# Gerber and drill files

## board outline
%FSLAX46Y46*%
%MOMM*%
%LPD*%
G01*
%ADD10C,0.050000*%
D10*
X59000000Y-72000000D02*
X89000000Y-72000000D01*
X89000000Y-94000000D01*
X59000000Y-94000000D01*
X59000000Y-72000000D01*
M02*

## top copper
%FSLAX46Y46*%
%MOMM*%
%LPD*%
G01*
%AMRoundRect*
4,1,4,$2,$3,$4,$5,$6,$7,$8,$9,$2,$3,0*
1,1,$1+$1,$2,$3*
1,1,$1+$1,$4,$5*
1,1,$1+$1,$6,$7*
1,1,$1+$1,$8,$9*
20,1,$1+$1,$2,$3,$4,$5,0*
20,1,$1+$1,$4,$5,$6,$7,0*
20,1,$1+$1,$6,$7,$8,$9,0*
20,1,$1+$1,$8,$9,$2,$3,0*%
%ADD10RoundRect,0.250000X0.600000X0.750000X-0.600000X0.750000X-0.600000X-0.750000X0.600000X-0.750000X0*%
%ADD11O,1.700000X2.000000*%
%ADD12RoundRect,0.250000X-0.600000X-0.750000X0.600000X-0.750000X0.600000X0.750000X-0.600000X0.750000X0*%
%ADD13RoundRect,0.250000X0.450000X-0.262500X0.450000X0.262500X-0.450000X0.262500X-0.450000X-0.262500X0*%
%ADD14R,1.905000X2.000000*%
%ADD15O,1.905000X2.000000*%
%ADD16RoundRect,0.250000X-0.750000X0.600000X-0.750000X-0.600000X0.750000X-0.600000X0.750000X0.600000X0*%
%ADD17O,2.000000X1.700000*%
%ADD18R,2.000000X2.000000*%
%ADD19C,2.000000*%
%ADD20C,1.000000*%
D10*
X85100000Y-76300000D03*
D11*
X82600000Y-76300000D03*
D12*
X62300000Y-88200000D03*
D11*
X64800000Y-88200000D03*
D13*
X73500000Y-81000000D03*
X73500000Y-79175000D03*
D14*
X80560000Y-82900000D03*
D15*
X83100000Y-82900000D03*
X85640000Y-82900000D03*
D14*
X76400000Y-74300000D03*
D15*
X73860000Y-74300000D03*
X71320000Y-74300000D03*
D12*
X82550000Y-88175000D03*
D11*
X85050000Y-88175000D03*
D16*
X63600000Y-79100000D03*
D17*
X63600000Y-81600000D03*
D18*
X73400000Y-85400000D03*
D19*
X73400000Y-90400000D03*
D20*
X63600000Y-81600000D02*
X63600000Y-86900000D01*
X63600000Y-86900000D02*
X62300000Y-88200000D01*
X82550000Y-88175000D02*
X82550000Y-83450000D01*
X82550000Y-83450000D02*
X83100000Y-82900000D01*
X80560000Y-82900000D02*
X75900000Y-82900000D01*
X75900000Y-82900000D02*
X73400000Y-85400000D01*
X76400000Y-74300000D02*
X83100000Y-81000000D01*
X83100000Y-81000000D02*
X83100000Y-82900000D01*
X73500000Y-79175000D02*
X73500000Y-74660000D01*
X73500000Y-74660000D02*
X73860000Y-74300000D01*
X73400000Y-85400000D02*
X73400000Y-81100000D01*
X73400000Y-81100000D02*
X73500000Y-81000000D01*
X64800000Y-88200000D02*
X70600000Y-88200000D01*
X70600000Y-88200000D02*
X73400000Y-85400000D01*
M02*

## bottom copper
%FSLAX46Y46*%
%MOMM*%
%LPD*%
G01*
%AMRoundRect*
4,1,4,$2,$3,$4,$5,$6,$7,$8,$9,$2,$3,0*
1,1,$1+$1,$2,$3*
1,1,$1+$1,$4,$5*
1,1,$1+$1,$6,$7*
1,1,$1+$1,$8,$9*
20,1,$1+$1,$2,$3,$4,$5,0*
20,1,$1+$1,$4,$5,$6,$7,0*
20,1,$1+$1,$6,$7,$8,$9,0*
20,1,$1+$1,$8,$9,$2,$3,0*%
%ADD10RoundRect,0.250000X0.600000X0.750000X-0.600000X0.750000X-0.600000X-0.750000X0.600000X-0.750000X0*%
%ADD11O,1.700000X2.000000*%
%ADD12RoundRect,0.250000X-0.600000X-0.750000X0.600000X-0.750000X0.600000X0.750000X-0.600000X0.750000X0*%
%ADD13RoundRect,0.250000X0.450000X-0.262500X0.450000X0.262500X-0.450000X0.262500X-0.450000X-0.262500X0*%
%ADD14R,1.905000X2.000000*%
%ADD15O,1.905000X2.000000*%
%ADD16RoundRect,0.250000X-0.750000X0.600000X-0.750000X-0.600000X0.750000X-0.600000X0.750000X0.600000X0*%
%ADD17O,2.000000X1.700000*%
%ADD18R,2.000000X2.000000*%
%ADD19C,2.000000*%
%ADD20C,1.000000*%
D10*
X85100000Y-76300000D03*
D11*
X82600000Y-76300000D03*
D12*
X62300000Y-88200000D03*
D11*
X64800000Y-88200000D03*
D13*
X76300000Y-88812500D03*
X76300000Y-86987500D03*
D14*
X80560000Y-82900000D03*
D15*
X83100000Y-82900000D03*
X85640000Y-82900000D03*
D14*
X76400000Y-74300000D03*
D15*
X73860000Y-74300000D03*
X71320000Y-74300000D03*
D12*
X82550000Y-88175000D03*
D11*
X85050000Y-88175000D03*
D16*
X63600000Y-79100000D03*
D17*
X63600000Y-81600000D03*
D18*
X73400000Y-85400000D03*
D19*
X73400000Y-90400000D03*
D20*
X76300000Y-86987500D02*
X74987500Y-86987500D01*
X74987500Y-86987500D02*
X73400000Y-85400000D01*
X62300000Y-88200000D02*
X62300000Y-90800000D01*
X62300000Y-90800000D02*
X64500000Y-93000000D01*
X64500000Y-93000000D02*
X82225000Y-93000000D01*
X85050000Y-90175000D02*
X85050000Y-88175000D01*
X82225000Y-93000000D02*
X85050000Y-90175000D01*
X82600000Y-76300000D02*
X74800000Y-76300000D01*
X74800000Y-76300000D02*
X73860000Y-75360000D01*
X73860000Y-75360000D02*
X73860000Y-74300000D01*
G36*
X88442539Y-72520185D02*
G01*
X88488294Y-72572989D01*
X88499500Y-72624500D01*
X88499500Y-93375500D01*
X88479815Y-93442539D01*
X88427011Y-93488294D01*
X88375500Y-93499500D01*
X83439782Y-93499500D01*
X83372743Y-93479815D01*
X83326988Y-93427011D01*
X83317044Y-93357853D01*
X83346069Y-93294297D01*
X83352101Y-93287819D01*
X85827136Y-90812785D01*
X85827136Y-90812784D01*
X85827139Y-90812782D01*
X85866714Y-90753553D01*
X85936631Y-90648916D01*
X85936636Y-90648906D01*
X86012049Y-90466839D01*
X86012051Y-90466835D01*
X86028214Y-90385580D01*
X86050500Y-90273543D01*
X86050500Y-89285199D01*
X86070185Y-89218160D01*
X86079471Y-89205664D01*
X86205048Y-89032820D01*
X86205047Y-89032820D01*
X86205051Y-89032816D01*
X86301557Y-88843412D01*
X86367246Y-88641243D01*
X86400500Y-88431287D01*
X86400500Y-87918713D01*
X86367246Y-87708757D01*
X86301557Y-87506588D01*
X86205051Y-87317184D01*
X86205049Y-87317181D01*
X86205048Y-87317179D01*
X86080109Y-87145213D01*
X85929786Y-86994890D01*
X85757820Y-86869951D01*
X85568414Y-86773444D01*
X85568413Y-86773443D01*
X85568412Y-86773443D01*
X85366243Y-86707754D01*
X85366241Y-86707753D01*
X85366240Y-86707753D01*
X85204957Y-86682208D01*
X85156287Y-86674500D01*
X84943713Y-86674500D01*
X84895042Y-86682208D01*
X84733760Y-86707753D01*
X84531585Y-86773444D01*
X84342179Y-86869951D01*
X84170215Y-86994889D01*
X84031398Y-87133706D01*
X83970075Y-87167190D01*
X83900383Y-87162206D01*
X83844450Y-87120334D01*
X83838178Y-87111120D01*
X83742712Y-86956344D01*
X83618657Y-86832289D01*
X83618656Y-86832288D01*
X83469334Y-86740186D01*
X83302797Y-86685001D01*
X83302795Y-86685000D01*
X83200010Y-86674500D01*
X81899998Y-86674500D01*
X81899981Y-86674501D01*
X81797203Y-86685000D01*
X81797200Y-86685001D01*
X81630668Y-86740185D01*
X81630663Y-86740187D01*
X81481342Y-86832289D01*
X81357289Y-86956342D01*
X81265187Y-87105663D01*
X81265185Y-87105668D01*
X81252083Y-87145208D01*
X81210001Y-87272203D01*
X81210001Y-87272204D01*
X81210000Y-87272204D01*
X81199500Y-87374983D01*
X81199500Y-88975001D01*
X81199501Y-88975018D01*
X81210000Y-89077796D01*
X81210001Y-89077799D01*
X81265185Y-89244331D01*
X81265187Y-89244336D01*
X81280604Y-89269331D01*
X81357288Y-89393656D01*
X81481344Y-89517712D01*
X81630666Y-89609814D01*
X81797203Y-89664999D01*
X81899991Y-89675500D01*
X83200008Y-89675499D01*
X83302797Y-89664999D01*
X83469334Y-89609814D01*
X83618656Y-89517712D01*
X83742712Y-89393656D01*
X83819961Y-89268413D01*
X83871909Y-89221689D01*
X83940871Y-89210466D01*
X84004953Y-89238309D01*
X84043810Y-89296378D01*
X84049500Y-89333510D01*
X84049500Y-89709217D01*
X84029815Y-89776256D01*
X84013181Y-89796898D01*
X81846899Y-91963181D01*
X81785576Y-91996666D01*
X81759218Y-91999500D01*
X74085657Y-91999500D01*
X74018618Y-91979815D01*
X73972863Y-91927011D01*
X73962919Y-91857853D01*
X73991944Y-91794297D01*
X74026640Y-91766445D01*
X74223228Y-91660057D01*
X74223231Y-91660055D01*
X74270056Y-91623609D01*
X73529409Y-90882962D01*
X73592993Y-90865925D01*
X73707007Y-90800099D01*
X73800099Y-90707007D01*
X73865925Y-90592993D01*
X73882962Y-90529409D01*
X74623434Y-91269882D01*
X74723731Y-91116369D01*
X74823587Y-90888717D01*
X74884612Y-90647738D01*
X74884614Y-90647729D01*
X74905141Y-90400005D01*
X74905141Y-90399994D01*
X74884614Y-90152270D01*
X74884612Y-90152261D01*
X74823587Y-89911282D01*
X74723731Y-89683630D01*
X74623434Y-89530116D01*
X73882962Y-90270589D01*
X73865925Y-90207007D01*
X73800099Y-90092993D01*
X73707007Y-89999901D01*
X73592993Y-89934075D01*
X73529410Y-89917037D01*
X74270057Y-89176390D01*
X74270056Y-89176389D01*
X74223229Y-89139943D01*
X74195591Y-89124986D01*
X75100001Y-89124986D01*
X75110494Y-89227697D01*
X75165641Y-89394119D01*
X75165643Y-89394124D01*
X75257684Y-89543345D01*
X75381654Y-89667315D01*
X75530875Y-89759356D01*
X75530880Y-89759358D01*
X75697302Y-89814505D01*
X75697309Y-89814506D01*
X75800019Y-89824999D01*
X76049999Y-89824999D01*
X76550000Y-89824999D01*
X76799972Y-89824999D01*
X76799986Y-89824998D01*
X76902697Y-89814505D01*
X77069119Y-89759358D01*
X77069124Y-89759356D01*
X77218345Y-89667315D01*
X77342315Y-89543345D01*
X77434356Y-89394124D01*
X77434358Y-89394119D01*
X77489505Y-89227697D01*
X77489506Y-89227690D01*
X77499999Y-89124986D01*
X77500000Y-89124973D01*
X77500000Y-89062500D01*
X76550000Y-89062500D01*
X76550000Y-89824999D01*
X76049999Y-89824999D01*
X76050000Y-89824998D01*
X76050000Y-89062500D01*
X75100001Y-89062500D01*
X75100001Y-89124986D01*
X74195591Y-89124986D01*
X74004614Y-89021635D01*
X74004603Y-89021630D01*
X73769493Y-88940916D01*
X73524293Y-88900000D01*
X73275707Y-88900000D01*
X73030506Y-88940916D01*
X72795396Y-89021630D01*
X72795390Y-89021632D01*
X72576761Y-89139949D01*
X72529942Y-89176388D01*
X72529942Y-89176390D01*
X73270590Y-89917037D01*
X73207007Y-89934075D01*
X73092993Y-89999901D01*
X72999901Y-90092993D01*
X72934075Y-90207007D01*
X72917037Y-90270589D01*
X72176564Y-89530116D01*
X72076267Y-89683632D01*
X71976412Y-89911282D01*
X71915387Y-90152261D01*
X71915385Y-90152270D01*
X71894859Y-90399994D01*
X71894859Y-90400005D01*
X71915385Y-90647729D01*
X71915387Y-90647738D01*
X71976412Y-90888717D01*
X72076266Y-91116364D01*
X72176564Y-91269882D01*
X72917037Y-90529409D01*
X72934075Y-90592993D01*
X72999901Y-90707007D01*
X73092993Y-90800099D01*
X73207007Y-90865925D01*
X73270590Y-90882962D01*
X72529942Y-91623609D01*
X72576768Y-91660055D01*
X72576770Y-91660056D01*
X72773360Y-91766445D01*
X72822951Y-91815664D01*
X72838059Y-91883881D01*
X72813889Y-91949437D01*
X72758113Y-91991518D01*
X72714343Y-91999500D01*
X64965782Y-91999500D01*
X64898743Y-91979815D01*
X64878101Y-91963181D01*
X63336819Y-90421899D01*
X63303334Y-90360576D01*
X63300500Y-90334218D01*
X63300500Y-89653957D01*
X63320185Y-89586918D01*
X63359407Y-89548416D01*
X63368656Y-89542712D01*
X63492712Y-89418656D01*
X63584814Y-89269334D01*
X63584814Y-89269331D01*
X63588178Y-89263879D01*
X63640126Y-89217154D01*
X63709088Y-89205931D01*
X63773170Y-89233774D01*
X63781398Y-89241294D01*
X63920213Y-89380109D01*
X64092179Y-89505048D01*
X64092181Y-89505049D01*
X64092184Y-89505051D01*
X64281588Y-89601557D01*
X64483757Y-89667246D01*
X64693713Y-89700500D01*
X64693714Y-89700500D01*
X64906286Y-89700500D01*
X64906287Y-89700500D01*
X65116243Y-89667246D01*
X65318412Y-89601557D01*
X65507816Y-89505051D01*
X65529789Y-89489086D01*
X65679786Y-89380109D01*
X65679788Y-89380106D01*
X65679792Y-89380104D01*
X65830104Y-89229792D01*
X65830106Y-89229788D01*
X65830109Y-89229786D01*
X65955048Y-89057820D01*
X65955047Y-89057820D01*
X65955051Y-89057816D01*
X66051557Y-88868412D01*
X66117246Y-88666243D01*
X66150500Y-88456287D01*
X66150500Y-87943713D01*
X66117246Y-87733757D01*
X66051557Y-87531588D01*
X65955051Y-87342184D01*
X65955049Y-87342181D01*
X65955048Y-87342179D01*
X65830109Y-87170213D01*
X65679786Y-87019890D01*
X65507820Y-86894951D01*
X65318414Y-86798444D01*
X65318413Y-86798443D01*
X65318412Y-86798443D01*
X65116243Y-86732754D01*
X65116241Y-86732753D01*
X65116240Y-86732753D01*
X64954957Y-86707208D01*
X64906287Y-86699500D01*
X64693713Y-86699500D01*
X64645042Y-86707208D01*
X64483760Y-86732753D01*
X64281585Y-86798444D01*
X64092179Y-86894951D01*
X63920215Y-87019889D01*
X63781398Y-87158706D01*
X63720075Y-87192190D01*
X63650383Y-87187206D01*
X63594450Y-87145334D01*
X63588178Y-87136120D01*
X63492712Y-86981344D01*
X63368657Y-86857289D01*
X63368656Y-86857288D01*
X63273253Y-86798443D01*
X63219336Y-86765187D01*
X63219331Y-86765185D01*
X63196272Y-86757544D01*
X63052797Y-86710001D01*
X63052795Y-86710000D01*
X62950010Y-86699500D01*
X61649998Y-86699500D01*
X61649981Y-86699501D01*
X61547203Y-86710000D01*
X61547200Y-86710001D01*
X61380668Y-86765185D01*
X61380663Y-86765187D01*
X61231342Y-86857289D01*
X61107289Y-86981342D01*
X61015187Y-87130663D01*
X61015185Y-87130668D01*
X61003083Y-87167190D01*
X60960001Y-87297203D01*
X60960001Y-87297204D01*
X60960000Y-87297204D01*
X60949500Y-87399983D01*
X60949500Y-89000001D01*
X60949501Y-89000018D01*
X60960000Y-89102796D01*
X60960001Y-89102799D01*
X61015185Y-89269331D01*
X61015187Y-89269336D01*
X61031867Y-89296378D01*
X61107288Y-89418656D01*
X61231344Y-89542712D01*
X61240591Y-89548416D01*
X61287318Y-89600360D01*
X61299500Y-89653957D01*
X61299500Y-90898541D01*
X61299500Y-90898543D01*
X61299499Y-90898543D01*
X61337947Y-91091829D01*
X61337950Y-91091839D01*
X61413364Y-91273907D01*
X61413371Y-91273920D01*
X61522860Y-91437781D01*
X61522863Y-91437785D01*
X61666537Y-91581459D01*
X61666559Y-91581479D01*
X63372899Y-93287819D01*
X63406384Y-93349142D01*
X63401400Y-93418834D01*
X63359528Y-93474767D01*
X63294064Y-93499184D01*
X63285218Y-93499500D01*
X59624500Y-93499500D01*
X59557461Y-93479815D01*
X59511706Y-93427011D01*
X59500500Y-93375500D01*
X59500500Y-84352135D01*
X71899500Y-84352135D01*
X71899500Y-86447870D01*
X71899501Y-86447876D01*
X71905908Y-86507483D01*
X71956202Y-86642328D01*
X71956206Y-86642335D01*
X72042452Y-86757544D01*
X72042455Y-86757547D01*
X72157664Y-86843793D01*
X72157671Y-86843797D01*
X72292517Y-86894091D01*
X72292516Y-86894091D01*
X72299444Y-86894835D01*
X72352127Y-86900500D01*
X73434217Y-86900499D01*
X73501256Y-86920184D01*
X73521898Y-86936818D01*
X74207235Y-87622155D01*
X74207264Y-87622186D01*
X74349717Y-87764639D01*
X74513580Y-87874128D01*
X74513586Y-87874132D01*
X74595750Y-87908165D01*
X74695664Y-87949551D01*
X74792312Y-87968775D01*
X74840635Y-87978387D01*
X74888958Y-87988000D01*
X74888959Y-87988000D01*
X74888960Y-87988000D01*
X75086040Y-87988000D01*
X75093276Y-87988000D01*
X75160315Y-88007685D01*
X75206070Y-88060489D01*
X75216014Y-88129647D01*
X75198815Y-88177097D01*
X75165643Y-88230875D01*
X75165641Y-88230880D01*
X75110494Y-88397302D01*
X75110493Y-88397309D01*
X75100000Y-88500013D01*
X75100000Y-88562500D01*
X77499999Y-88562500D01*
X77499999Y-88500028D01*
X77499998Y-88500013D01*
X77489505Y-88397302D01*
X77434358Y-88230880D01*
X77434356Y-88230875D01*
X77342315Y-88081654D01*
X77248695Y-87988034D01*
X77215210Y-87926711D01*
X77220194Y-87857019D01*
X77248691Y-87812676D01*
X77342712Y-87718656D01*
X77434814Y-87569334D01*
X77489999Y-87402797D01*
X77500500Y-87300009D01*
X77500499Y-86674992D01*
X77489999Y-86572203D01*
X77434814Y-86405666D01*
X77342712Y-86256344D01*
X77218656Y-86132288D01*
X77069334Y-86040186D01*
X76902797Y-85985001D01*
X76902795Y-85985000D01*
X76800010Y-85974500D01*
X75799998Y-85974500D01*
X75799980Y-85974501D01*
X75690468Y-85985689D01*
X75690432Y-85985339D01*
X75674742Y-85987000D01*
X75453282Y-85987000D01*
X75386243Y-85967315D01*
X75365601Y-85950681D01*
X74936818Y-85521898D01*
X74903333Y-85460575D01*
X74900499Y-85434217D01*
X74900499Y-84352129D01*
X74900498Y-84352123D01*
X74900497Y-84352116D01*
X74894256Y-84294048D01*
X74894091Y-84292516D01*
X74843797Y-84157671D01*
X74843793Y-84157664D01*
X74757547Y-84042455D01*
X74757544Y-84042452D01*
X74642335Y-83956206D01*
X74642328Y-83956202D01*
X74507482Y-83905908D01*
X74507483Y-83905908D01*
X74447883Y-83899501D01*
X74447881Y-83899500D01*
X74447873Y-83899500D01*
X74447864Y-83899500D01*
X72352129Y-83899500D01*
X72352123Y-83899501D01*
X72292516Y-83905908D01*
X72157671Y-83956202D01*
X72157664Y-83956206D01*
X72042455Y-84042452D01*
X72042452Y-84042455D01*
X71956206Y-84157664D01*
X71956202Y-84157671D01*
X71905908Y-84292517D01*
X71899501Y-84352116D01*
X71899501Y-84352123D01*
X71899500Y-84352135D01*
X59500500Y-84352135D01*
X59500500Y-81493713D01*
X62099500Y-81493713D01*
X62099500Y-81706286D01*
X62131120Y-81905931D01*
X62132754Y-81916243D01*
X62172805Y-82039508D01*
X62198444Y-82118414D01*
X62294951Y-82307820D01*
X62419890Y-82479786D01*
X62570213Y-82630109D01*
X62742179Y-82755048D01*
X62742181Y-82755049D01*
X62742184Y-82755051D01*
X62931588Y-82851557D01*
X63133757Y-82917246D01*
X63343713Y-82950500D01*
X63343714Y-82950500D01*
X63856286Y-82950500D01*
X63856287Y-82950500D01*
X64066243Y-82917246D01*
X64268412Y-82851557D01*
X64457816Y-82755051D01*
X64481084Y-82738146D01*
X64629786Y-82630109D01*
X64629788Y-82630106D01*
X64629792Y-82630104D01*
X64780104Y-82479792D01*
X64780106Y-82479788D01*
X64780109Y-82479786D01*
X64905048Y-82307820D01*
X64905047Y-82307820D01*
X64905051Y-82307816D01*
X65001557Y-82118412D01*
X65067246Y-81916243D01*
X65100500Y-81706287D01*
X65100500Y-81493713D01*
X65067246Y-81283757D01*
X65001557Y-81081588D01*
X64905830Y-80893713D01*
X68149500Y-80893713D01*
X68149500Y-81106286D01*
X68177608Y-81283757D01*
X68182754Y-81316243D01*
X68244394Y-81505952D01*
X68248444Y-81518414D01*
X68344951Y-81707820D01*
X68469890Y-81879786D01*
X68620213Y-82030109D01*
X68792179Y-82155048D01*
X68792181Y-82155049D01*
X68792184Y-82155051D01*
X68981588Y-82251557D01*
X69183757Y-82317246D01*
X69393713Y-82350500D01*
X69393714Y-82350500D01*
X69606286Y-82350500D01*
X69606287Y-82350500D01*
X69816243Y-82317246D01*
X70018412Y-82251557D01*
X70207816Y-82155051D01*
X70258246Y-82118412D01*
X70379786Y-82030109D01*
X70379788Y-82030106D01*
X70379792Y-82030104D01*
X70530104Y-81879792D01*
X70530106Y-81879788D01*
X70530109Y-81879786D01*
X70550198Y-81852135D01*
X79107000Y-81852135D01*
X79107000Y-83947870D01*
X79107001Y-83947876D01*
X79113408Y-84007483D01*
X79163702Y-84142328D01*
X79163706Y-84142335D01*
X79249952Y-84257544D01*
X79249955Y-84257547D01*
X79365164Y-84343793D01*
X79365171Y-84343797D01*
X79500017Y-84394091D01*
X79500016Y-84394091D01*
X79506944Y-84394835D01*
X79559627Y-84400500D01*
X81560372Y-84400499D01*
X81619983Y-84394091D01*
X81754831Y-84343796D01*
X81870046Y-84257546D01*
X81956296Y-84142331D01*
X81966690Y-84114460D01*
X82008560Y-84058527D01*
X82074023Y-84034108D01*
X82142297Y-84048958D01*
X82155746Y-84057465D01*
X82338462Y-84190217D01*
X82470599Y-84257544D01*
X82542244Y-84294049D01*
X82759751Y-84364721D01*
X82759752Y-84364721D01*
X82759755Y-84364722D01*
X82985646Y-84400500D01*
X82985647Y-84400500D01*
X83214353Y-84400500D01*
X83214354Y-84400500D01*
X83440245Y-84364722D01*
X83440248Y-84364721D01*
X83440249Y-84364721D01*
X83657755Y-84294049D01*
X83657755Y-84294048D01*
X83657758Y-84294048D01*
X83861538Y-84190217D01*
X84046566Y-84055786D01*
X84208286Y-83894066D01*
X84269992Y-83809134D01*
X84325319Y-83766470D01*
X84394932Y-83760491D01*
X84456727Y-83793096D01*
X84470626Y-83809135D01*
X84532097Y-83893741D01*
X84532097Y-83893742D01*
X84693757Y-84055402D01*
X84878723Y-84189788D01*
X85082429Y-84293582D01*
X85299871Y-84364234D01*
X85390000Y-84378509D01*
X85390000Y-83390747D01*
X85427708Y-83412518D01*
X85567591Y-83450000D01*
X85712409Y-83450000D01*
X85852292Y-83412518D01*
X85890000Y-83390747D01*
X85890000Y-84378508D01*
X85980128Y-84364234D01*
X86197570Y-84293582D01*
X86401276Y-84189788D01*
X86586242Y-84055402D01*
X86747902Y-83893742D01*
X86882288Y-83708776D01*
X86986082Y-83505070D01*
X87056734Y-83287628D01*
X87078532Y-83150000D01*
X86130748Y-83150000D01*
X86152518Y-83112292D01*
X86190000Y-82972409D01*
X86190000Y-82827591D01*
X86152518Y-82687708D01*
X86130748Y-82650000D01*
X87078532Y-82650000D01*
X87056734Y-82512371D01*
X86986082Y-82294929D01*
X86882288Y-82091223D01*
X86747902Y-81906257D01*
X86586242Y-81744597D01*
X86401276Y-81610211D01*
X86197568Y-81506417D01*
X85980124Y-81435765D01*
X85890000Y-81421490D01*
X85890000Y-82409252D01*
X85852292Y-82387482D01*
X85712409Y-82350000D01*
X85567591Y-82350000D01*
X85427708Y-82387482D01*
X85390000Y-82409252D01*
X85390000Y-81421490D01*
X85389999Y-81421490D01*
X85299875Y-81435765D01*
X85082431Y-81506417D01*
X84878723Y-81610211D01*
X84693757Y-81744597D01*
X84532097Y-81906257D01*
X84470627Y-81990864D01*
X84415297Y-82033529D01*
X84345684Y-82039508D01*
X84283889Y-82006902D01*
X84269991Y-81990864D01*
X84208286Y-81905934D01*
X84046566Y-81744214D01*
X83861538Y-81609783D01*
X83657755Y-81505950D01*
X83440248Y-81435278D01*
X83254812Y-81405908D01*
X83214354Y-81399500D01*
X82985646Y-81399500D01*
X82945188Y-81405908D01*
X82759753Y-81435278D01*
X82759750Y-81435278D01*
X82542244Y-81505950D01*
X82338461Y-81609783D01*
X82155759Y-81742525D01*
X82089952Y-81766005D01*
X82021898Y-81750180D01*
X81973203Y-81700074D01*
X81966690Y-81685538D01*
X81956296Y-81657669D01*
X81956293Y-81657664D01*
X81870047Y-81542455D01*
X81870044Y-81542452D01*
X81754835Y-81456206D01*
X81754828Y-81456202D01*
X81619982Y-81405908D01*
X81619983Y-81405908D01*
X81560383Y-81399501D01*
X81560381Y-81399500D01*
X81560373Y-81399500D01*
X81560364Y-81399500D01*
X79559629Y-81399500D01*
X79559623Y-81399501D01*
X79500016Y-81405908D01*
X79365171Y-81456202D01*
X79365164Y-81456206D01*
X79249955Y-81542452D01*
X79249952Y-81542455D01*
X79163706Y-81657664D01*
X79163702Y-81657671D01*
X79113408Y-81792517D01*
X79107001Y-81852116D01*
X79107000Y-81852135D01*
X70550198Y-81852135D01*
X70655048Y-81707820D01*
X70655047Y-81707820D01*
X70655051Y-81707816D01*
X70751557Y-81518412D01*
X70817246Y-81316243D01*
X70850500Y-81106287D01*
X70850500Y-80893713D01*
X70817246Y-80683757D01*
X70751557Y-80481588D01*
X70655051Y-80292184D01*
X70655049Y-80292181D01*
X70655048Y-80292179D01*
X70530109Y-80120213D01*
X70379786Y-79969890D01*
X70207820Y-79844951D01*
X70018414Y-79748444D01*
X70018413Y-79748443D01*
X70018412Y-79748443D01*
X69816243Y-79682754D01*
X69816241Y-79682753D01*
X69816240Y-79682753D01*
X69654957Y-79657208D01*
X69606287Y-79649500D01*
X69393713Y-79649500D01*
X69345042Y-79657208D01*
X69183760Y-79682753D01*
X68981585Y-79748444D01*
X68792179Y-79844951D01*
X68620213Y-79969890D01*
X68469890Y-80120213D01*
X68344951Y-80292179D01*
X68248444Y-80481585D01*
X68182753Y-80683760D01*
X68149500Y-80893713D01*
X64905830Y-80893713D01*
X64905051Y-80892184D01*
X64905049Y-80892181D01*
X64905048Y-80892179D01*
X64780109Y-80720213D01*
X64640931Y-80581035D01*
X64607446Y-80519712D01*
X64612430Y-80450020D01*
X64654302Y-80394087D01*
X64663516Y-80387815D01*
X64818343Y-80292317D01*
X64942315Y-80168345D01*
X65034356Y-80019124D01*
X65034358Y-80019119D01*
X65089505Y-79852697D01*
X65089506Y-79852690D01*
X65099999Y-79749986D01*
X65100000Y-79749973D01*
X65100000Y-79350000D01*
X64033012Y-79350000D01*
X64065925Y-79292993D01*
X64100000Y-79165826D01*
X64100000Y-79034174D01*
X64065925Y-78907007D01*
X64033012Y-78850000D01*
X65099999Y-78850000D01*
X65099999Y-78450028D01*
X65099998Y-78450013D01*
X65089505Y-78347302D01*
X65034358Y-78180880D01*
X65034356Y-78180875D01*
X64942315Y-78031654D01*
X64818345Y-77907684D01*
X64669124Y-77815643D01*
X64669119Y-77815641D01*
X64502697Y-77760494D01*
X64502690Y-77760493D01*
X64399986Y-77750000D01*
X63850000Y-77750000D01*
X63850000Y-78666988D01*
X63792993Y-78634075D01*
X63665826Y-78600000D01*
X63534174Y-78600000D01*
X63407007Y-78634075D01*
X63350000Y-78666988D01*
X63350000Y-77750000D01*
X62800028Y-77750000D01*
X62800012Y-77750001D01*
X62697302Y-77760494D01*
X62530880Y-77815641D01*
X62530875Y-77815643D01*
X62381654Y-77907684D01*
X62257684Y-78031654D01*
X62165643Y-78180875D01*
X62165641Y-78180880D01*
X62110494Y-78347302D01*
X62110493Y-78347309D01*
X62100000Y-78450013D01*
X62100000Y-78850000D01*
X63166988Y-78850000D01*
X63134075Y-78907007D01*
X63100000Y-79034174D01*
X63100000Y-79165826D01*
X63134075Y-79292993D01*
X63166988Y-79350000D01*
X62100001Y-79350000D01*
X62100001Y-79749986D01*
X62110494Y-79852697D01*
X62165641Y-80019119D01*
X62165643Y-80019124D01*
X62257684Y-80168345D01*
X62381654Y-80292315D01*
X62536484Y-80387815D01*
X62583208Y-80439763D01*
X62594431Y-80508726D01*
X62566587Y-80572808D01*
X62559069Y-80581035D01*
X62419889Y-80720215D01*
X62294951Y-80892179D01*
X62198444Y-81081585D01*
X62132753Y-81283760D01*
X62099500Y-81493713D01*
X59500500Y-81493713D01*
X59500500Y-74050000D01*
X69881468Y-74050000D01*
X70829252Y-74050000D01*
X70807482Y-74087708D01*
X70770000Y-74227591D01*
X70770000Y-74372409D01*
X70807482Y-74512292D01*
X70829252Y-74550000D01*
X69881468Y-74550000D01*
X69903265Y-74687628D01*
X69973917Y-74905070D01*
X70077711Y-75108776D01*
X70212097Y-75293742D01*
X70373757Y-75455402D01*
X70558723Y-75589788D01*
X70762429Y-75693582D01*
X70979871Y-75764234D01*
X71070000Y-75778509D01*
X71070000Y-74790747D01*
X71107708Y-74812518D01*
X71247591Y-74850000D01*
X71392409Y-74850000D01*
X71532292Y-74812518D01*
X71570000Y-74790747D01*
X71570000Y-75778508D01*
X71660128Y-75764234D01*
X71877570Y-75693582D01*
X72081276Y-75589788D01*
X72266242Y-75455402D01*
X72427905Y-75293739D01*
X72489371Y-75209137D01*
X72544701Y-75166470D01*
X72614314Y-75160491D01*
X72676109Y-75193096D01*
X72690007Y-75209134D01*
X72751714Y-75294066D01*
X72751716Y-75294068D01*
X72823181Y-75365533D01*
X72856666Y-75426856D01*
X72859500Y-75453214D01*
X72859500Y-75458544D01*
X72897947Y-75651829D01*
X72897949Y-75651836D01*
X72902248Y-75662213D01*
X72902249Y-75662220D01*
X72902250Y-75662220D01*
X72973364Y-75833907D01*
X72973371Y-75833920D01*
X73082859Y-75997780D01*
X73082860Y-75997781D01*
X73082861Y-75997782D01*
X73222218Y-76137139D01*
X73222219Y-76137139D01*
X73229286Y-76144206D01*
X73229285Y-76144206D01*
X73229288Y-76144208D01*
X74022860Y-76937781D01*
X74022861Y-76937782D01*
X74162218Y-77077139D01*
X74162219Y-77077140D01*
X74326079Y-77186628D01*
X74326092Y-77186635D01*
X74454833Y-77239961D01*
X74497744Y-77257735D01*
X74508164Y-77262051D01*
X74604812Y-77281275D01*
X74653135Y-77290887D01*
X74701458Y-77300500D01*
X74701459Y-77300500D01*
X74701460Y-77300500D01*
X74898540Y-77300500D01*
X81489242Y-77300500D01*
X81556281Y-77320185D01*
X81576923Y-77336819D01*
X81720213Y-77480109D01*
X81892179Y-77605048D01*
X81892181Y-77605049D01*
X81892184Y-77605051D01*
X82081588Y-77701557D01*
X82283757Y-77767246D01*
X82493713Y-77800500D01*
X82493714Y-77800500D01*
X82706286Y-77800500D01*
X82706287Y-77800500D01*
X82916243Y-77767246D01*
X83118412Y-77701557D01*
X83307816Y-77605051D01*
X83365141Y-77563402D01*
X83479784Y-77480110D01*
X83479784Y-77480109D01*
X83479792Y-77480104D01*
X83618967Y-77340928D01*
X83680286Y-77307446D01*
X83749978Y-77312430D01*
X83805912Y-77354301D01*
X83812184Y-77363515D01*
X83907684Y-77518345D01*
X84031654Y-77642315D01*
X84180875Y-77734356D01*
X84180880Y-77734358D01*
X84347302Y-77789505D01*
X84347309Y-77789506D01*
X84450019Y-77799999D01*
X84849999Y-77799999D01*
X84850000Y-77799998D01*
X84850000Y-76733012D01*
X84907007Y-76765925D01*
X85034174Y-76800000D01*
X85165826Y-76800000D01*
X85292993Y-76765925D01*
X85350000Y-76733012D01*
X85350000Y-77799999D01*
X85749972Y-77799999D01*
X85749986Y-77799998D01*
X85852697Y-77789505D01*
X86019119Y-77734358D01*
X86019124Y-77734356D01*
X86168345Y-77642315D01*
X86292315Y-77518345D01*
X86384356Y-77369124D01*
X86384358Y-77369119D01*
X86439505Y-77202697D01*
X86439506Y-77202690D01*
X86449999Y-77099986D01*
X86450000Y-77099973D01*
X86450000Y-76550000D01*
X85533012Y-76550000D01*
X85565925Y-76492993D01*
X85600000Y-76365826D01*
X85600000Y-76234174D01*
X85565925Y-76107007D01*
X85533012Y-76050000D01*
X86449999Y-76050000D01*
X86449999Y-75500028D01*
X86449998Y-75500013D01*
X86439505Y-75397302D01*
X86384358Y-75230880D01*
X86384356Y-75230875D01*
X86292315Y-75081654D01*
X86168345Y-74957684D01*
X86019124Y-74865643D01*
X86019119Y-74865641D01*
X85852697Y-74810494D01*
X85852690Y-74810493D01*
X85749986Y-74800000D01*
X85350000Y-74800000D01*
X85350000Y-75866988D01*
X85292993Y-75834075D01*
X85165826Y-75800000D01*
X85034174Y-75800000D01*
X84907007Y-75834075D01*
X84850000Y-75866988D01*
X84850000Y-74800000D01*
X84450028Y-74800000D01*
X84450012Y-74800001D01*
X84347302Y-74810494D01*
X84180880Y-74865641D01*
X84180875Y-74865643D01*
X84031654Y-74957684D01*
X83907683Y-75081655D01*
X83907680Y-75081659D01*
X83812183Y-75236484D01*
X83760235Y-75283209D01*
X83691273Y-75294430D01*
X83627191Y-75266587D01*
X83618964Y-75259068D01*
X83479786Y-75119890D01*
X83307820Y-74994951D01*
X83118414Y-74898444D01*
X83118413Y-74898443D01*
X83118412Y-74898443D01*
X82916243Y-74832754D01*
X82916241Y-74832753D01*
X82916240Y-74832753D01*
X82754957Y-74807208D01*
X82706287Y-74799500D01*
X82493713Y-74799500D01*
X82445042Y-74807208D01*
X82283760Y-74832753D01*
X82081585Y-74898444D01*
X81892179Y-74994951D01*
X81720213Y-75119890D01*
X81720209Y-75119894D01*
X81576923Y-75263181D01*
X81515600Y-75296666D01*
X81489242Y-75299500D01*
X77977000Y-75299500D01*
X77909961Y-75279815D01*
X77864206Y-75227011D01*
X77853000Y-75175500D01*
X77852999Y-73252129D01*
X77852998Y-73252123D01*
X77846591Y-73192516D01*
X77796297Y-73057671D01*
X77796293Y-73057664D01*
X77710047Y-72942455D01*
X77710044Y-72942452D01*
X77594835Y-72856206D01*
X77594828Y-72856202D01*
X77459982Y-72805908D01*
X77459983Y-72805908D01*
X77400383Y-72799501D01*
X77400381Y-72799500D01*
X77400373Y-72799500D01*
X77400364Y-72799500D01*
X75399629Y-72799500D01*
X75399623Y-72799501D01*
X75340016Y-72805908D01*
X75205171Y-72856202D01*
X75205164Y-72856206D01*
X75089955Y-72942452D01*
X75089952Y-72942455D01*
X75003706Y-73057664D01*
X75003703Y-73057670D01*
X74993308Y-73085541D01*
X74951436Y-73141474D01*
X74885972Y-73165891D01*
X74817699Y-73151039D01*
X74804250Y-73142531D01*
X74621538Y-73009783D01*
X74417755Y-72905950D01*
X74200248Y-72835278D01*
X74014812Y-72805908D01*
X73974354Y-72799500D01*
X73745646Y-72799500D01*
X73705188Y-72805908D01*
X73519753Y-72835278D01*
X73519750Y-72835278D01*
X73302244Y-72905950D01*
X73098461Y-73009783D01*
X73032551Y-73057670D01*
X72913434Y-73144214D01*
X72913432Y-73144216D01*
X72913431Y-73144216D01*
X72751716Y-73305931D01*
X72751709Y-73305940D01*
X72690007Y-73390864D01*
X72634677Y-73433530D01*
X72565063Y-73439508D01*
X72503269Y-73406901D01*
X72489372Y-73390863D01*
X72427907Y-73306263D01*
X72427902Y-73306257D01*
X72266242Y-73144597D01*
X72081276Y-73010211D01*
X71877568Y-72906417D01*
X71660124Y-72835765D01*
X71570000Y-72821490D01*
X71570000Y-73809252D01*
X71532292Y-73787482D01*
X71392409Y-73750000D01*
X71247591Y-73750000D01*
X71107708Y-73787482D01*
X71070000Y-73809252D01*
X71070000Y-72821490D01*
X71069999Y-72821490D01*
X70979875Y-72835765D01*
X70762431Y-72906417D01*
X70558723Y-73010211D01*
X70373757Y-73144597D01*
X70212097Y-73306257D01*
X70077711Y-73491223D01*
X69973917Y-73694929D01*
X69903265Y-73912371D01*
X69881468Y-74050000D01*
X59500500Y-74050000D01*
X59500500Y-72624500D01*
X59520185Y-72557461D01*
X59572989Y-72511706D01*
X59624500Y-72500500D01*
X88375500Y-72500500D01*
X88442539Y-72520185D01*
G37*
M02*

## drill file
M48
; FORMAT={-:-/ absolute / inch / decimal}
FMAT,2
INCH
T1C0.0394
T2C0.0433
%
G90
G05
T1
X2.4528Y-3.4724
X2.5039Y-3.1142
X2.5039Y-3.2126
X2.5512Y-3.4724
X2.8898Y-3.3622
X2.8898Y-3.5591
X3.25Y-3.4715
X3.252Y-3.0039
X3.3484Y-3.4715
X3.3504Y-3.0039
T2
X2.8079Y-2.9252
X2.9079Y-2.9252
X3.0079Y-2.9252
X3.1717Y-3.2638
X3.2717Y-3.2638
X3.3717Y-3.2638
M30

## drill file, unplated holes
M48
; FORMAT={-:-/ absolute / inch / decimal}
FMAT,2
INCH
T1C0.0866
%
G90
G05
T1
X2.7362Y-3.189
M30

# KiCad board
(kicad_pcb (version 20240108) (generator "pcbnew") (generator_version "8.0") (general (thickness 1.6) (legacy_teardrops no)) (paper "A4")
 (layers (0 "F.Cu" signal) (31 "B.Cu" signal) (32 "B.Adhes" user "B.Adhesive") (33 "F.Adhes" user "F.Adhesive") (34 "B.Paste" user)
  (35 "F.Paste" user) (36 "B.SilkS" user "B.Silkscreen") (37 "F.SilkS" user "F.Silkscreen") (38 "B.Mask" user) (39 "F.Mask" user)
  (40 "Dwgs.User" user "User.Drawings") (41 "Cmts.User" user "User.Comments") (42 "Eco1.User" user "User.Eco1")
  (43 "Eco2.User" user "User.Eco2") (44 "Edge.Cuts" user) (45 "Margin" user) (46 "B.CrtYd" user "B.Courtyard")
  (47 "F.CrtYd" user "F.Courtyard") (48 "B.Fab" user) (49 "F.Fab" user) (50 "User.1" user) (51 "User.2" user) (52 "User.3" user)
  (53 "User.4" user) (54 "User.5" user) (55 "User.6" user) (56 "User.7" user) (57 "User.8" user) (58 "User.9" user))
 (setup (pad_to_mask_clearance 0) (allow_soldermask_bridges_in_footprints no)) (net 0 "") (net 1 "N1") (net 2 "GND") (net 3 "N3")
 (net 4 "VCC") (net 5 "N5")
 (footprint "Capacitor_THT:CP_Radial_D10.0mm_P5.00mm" (layer "F.Cu") (at 73.4 85.4 -90)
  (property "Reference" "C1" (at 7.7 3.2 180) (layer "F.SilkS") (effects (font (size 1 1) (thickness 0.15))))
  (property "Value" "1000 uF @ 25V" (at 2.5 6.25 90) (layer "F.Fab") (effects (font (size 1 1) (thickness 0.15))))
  (pad "1" thru_hole rect (at 0 0 270) (size 2 2) (drill 1) (layers "*.Cu" "*.Mask") (remove_unused_layers no) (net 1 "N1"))
  (pad "2" thru_hole circle (at 5 0 270) (size 2 2) (drill 1) (layers "*.Cu" "*.Mask") (remove_unused_layers no) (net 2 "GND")))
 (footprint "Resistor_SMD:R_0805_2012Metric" (layer "F.Cu") (at 73.5 80.0875 90)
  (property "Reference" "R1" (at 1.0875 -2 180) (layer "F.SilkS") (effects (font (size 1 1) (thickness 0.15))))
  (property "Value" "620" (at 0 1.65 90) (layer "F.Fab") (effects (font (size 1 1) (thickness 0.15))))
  (pad "1" smd roundrect (at -0.9125 0 90) (size 1.025 1.4) (layers "F.Cu" "F.Paste" "F.Mask") (roundrect_rratio 0.243902) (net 1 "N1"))
  (pad "2" smd roundrect (at 0.9125 0 90) (size 1.025 1.4) (layers "F.Cu" "F.Paste" "F.Mask") (roundrect_rratio 0.243902) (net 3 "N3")))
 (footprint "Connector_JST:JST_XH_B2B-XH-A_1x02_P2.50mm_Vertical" (layer "F.Cu") (at 63.6 79.1 -90)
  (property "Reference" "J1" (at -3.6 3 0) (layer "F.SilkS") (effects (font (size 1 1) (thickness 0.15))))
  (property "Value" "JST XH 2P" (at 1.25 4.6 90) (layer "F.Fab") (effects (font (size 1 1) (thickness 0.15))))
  (pad "1" thru_hole roundrect (at 0 0 270) (size 1.7 2) (drill 1) (layers "*.Cu" "*.Mask") (remove_unused_layers no)
   (roundrect_rratio 0.147059) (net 2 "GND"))
  (pad "2" thru_hole oval (at 2.5 0 270) (size 1.7 2) (drill 1) (layers "*.Cu" "*.Mask") (remove_unused_layers no) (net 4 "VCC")))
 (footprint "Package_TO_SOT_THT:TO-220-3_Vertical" (layer "F.Cu") (at 80.56 82.9)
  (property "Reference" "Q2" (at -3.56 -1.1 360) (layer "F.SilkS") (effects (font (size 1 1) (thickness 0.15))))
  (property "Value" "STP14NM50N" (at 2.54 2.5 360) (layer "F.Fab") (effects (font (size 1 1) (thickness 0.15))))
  (pad "1" thru_hole rect (at 0 0) (size 1.905 2) (drill 1.1) (layers "*.Cu" "*.Mask") (remove_unused_layers no) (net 1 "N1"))
  (pad "2" thru_hole oval (at 2.54 0) (size 1.905 2) (drill 1.1) (layers "*.Cu" "*.Mask") (remove_unused_layers no) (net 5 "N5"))
  (pad "3" thru_hole oval (at 5.08 0) (size 1.905 2) (drill 1.1) (layers "*.Cu" "*.Mask") (remove_unused_layers no) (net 2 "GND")))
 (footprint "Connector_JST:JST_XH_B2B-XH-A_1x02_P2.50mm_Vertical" (layer "F.Cu") (at 62.3 88.2)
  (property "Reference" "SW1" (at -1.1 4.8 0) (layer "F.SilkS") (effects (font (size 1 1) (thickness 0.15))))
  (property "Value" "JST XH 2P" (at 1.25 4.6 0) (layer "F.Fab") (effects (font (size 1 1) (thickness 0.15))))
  (pad "1" thru_hole roundrect (at 0 0) (size 1.7 2) (drill 1) (layers "*.Cu" "*.Mask") (remove_unused_layers no)
   (roundrect_rratio 0.147059) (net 4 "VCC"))
  (pad "2" thru_hole oval (at 2.5 0) (size 1.7 2) (drill 1) (layers "*.Cu" "*.Mask") (remove_unused_layers no) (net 1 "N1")))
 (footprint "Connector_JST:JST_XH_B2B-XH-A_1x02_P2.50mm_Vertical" (layer "F.Cu") (at 82.55 88.175)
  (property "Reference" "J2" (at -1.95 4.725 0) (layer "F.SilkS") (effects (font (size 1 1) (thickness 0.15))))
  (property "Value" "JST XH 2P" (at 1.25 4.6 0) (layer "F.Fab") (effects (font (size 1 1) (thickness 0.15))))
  (pad "1" thru_hole roundrect (at 0 0) (size 1.7 2) (drill 1) (layers "*.Cu" "*.Mask") (remove_unused_layers no)
   (roundrect_rratio 0.147059) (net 5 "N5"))
  (pad "2" thru_hole oval (at 2.5 0) (size 1.7 2) (drill 1) (layers "*.Cu" "*.Mask") (remove_unused_layers no) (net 4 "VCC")))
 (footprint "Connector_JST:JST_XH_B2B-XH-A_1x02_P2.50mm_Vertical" (layer "F.Cu") (at 85.1 76.3 180)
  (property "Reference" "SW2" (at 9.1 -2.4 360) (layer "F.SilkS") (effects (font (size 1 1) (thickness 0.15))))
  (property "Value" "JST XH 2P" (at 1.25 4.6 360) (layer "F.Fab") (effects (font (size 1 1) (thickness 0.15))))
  (pad "1" thru_hole roundrect (at 0 0 180) (size 1.7 2) (drill 1) (layers "*.Cu" "*.Mask") (remove_unused_layers no)
   (roundrect_rratio 0.147059) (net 2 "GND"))
  (pad "2" thru_hole oval (at 2.5 0 180) (size 1.7 2) (drill 1) (layers "*.Cu" "*.Mask") (remove_unused_layers no) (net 3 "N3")))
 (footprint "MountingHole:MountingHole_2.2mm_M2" (layer "F.Cu") (at 69.5 81)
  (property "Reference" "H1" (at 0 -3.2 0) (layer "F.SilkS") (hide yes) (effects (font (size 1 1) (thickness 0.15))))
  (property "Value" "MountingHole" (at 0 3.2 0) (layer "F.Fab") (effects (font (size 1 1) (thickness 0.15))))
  (pad "" np_thru_hole circle (at 0 0) (size 2.2 2.2) (drill 2.2) (layers "*.Cu" "*.Mask")))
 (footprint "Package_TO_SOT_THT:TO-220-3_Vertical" (layer "F.Cu") (at 76.4 74.3 180)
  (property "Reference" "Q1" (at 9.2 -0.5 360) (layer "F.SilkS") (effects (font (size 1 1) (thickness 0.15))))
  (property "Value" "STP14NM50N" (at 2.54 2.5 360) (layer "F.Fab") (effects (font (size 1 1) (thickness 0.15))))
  (pad "1" thru_hole rect (at 0 0 180) (size 1.905 2) (drill 1.1) (layers "*.Cu" "*.Mask") (remove_unused_layers no) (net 5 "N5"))
  (pad "2" thru_hole oval (at 2.54 0 180) (size 1.905 2) (drill 1.1) (layers "*.Cu" "*.Mask") (remove_unused_layers no) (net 3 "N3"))
  (pad "3" thru_hole oval (at 5.08 0 180) (size 1.905 2) (drill 1.1) (layers "*.Cu" "*.Mask") (remove_unused_layers no) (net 2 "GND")))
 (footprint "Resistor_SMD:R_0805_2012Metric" (layer "B.Cu") (at 76.3 87.9 90)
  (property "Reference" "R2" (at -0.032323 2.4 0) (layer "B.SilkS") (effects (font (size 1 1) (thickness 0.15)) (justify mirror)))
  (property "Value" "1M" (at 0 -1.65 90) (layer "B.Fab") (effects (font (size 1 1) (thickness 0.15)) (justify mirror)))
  (pad "1" smd roundrect (at -0.9125 0 90) (size 1.025 1.4) (layers "B.Cu" "B.Paste" "B.Mask") (roundrect_rratio 0.243902) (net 2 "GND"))
  (pad "2" smd roundrect (at 0.9125 0 90) (size 1.025 1.4) (layers "B.Cu" "B.Paste" "B.Mask") (roundrect_rratio 0.243902) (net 1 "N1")))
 (gr_rect (start 59 72) (end 89 94) (stroke (width 0.05) (type default)) (fill none) (layer "Edge.Cuts"))
 (segment (start 70.6 88.2) (end 73.4 85.4) (width 1) (layer "F.Cu") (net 1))
 (segment (start 73.4 85.4) (end 73.4 81.1) (width 1) (layer "F.Cu") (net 1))
 (segment (start 80.56 82.9) (end 75.9 82.9) (width 1) (layer "F.Cu") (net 1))
 (segment (start 73.4 81.1) (end 73.5 81) (width 1) (layer "F.Cu") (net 1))
 (segment (start 75.9 82.9) (end 73.4 85.4) (width 1) (layer "F.Cu") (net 1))
 (segment (start 64.8 88.2) (end 70.6 88.2) (width 1) (layer "F.Cu") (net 1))
 (segment (start 76.3 86.9875) (end 74.9875 86.9875) (width 1) (layer "B.Cu") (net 1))
 (segment (start 74.9875 86.9875) (end 73.4 85.4) (width 1) (layer "B.Cu") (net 1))
 (segment (start 63.6 81.6) (end 63.6 86.9) (width 1) (layer "F.Cu") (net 4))
 (segment (start 63.6 86.9) (end 62.3 88.2) (width 1) (layer "F.Cu") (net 4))
 (segment (start 62.3 90.8) (end 64.5 93) (width 1) (layer "B.Cu") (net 4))
 (segment (start 62.3 88.2) (end 62.3 90.8) (width 1) (layer "B.Cu") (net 4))
 (segment (start 82.225 93) (end 85.05 90.175) (width 1) (layer "B.Cu") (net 4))
 (segment (start 85.05 90.175) (end 85.05 88.175) (width 1) (layer "B.Cu") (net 4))
 (segment (start 64.5 93) (end 82.225 93) (width 1) (layer "B.Cu") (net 4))
 (segment (start 82.55 88.175) (end 82.55 83.45) (width 1) (layer "F.Cu") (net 5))
 (segment (start 76.4 74.3) (end 83.1 81) (width 1) (layer "F.Cu") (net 5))
 (segment (start 83.1 81) (end 83.1 82.9) (width 1) (layer "F.Cu") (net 5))
 (segment (start 82.55 83.45) (end 83.1 82.9) (width 1) (layer "F.Cu") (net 5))
 (segment (start 73.5 79.175) (end 73.5 74.66) (width 1) (layer "F.Cu") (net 3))
 (segment (start 73.5 74.66) (end 73.86 74.3) (width 1) (layer "F.Cu") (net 3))
 (segment (start 82.6 76.3) (end 74.8 76.3) (width 1) (layer "B.Cu") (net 3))
 (segment (start 73.86 75.36) (end 73.86 74.3) (width 1) (layer "B.Cu") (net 3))
 (segment (start 74.8 76.3) (end 73.86 75.36) (width 1) (layer "B.Cu") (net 3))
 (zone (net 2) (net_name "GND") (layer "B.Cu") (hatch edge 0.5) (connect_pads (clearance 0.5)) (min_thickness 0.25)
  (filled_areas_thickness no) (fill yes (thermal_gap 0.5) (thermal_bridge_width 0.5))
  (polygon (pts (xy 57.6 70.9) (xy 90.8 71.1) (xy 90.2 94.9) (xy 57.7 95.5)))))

